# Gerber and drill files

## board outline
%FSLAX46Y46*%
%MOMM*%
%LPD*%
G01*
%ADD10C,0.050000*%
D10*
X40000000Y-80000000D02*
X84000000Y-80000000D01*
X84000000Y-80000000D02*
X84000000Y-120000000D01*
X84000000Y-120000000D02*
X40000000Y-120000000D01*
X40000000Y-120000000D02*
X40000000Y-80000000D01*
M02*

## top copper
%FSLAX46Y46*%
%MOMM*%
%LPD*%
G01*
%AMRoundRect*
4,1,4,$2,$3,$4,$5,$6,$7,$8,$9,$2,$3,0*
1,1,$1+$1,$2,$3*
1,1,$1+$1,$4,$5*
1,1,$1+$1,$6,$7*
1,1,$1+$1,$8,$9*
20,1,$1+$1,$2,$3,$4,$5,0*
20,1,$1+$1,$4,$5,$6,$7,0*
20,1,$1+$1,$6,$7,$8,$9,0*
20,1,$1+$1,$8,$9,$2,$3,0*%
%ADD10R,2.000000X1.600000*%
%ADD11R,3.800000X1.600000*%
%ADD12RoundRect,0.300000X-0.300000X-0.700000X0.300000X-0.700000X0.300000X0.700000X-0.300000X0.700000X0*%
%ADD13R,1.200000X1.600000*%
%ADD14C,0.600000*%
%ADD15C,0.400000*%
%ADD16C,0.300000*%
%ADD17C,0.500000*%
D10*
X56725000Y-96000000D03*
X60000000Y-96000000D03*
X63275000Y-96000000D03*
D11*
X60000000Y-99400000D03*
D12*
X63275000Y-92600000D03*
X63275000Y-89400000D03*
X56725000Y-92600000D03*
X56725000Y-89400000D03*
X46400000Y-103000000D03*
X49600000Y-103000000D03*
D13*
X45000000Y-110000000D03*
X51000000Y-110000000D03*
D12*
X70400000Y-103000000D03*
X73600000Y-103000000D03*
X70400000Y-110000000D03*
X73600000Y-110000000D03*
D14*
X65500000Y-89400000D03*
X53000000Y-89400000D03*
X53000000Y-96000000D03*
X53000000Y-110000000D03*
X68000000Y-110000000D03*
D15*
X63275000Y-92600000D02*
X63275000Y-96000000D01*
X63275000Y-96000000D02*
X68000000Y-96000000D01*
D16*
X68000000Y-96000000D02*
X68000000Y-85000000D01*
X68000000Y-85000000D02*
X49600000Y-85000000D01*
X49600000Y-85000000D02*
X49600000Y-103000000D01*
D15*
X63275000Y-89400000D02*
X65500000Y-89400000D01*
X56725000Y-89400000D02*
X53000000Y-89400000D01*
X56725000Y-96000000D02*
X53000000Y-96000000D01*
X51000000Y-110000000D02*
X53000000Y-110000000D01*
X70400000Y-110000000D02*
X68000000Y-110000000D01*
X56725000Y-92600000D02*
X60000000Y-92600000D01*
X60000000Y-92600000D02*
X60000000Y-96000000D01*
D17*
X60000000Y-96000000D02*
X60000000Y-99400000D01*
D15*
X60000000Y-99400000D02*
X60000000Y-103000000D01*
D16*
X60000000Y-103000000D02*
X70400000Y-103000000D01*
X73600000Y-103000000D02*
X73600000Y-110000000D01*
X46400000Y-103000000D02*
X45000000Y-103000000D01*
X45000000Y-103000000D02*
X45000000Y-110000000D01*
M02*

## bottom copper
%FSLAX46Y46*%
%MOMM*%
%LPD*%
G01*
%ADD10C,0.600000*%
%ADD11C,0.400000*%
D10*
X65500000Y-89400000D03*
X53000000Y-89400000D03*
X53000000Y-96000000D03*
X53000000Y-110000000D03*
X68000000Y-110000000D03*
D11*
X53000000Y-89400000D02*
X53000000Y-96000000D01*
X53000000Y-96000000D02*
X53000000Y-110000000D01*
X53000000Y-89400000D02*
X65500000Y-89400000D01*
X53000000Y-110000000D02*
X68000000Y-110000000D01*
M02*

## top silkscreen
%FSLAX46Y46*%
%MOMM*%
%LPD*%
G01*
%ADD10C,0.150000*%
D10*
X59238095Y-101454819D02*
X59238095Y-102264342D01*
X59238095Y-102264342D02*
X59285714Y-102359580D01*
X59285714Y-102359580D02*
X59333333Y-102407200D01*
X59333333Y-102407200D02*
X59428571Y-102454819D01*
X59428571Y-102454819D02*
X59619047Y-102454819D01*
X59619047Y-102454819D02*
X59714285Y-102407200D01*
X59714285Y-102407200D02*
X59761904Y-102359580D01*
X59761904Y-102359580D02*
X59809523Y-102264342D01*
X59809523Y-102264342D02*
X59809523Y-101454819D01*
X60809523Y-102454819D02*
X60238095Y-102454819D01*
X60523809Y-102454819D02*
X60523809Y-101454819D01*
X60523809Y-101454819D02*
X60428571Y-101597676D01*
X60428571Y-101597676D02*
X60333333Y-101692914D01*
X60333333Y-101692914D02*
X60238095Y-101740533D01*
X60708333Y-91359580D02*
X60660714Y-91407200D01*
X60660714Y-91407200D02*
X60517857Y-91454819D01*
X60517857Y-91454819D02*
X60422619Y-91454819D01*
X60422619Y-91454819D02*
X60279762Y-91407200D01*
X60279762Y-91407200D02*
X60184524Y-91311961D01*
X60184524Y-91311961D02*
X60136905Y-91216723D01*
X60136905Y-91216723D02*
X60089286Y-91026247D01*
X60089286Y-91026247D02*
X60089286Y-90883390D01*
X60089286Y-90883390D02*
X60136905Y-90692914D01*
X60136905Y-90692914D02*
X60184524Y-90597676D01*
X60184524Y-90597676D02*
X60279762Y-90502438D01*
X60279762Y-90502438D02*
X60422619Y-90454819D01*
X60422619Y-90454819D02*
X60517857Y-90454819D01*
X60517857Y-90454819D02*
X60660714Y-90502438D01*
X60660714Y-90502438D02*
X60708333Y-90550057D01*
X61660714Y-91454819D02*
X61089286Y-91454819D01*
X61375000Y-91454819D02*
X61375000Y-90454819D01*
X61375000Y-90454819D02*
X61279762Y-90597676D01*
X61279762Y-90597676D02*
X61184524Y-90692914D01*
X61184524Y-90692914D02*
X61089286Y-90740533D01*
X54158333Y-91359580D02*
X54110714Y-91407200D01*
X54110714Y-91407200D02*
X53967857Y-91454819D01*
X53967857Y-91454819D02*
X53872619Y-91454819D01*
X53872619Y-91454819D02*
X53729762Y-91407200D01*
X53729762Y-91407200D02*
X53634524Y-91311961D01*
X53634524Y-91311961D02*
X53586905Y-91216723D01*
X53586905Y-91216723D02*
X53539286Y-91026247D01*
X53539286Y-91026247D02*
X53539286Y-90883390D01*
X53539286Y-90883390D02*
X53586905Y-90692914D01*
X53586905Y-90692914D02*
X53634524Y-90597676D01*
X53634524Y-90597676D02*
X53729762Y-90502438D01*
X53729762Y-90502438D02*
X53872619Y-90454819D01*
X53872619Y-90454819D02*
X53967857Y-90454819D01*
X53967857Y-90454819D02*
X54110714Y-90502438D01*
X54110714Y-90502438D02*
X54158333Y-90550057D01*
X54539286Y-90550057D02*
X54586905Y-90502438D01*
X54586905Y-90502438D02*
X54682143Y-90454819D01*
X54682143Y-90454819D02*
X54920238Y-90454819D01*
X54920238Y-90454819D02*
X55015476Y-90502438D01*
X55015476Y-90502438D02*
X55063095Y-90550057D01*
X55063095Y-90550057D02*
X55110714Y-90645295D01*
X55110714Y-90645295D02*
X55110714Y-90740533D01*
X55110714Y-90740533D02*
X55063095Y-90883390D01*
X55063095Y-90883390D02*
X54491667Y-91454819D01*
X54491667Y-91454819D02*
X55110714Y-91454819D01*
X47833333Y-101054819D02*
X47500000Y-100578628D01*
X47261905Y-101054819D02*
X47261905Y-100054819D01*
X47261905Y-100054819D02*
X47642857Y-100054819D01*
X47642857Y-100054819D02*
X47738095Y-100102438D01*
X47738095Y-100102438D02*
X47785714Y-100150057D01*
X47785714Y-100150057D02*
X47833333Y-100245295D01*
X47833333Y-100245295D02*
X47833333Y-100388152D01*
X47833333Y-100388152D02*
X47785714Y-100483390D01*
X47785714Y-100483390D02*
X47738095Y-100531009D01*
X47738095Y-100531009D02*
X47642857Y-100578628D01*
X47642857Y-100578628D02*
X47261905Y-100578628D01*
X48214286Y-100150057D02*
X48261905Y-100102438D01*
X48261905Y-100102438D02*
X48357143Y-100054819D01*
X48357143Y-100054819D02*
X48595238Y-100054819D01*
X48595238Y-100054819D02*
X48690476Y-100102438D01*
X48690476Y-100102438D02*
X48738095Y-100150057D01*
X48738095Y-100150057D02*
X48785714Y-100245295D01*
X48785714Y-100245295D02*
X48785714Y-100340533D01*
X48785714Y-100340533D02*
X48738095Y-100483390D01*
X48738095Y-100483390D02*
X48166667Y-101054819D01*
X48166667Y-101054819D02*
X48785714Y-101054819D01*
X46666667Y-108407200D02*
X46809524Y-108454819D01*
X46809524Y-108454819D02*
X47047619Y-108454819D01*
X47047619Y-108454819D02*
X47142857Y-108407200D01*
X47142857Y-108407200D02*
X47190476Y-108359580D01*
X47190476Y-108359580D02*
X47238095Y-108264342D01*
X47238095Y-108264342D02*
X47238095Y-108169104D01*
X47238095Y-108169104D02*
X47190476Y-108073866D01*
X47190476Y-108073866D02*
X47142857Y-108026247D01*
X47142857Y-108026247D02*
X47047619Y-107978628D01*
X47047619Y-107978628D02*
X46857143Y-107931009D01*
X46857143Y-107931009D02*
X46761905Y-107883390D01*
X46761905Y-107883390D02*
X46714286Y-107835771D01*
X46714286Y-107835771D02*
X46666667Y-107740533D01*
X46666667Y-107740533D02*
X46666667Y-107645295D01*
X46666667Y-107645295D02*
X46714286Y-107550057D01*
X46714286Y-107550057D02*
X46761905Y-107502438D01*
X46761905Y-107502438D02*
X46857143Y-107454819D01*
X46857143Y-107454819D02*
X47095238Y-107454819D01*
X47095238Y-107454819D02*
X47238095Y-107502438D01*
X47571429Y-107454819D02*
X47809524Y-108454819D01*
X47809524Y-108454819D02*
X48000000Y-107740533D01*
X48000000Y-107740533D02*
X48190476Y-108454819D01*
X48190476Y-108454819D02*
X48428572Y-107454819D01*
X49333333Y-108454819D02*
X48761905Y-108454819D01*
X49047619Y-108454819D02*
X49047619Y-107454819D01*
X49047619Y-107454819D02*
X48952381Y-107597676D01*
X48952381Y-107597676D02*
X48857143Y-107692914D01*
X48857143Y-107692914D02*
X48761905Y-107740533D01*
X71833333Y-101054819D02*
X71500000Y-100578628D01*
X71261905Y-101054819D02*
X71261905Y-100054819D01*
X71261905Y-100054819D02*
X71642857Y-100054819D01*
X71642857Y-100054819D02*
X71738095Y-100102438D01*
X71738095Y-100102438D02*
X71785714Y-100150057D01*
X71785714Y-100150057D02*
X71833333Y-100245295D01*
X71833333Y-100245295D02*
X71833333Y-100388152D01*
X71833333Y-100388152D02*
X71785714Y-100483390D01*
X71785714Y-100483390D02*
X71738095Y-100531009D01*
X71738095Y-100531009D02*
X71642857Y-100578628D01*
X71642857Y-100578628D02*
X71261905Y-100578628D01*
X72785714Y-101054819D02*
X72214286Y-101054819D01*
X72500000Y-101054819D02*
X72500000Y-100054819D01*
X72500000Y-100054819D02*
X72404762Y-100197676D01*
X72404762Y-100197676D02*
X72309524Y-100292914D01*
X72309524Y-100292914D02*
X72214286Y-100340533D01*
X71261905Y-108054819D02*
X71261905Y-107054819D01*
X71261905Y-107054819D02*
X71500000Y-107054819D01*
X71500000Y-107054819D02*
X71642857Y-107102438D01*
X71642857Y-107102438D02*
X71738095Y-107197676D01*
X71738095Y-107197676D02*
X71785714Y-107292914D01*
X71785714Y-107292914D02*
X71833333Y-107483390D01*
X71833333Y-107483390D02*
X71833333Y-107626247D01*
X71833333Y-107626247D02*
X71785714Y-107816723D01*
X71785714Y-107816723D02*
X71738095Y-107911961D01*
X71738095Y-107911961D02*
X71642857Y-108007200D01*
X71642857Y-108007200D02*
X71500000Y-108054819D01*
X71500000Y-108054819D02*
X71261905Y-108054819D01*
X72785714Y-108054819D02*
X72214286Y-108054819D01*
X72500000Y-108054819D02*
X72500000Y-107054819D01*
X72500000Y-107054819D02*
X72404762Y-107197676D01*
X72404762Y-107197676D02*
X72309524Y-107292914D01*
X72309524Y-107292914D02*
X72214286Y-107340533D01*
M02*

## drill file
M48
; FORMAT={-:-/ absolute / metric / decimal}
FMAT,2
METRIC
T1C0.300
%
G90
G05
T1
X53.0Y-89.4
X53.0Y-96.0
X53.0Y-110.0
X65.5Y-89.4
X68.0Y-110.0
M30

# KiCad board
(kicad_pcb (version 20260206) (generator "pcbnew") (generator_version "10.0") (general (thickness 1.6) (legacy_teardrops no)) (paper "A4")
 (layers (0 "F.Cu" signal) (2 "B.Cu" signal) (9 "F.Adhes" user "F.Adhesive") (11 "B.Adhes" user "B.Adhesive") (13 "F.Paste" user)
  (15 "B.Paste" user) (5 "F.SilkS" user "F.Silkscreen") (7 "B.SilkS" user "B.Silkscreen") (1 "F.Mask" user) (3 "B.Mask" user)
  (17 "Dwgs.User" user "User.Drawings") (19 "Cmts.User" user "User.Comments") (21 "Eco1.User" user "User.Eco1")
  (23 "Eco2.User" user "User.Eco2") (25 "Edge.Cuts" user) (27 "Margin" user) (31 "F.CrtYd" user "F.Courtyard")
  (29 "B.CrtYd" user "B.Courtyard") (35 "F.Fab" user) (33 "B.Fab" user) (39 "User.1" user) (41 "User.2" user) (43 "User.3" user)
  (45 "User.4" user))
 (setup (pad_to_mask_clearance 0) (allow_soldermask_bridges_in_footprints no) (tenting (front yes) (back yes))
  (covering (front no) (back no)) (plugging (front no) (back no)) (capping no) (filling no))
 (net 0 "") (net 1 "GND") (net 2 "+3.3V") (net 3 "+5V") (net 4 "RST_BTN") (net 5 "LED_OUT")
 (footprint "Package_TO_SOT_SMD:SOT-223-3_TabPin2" (layer "F.Cu") (at 60 96)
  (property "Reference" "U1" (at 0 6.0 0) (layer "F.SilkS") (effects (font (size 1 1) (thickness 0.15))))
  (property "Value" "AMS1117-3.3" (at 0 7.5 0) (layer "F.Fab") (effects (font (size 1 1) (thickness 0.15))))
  (pad "1" smd rect (at -3.275 0) (size 2 1.6) (layers "F.Cu" "F.Paste" "F.Mask") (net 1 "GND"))
  (pad "2" smd rect (at 0 0) (size 2 1.6) (layers "F.Cu" "F.Paste" "F.Mask") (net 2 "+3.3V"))
  (pad "3" smd rect (at 3.275 0) (size 2 1.6) (layers "F.Cu" "F.Paste" "F.Mask") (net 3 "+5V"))
  (pad "2" smd rect (at 0 3.4) (size 3.8 1.6) (layers "F.Cu" "F.Paste" "F.Mask") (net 2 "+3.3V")))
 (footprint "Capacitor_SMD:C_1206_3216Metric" (layer "F.Cu") (at 63.275 91 90)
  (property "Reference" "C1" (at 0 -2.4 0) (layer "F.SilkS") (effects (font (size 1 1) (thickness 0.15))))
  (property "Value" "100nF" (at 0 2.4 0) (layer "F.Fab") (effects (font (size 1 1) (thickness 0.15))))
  (pad "1" smd roundrect (at -1.6 0) (size 1.2 2) (layers "F.Cu" "F.Paste" "F.Mask") (roundrect_rratio 0.25) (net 3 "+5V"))
  (pad "2" smd roundrect (at 1.6 0) (size 1.2 2) (layers "F.Cu" "F.Paste" "F.Mask") (roundrect_rratio 0.25) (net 1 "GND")))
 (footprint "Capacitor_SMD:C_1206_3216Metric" (layer "F.Cu") (at 56.725 91 90)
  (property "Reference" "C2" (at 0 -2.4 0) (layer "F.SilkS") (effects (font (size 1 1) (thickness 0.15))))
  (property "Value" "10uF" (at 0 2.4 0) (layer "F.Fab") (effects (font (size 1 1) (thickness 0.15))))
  (pad "1" smd roundrect (at -1.6 0) (size 1.2 2) (layers "F.Cu" "F.Paste" "F.Mask") (roundrect_rratio 0.25) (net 2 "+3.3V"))
  (pad "2" smd roundrect (at 1.6 0) (size 1.2 2) (layers "F.Cu" "F.Paste" "F.Mask") (roundrect_rratio 0.25) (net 1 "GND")))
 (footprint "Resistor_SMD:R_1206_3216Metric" (layer "F.Cu") (at 48 103)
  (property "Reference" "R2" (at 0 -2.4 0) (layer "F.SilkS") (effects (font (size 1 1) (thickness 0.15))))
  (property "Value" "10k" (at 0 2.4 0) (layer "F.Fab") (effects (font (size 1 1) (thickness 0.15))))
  (pad "2" smd roundrect (at -1.6 0) (size 1.2 2) (layers "F.Cu" "F.Paste" "F.Mask") (roundrect_rratio 0.25) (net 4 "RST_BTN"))
  (pad "1" smd roundrect (at 1.6 0) (size 1.2 2) (layers "F.Cu" "F.Paste" "F.Mask") (roundrect_rratio 0.25) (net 3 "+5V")))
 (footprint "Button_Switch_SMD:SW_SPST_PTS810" (layer "F.Cu") (at 48 110)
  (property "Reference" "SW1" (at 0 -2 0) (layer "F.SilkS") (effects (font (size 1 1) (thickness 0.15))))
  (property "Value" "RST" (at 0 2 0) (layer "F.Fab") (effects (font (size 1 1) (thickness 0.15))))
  (pad "1" smd rect (at -3 0) (size 1.2 1.6) (layers "F.Cu" "F.Paste" "F.Mask") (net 4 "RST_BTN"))
  (pad "2" smd rect (at 3 0) (size 1.2 1.6) (layers "F.Cu" "F.Paste" "F.Mask") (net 1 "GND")))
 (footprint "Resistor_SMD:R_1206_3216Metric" (layer "F.Cu") (at 72 103)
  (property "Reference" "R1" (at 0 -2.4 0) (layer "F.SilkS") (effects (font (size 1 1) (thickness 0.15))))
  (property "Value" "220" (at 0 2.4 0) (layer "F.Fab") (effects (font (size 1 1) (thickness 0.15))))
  (pad "1" smd roundrect (at -1.6 0) (size 1.2 2) (layers "F.Cu" "F.Paste" "F.Mask") (roundrect_rratio 0.25) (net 2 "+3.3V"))
  (pad "2" smd roundrect (at 1.6 0) (size 1.2 2) (layers "F.Cu" "F.Paste" "F.Mask") (roundrect_rratio 0.25) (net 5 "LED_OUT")))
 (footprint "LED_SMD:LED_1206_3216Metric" (layer "F.Cu") (at 72 110)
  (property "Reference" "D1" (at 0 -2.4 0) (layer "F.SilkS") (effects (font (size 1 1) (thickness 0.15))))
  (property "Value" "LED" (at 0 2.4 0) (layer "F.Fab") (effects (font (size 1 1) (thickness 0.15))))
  (pad "2" smd roundrect (at -1.6 0) (size 1.2 2) (layers "F.Cu" "F.Paste" "F.Mask") (roundrect_rratio 0.25) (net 1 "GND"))
  (pad "1" smd roundrect (at 1.6 0) (size 1.2 2) (layers "F.Cu" "F.Paste" "F.Mask") (roundrect_rratio 0.25) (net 5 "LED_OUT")))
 (segment (start 63.275 92.6) (end 63.275 96) (width 0.4) (layer "F.Cu") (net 3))
 (segment (start 63.275 96) (end 68 96) (width 0.4) (layer "F.Cu") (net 3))
 (segment (start 68 96) (end 68 85) (width 0.3) (layer "F.Cu") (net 3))
 (segment (start 68 85) (end 49.6 85) (width 0.3) (layer "F.Cu") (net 3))
 (segment (start 49.6 85) (end 49.6 103) (width 0.3) (layer "F.Cu") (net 3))
 (segment (start 63.275 89.4) (end 65.5 89.4) (width 0.4) (layer "F.Cu") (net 1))
 (via (at 65.5 89.4) (size 0.6) (drill 0.3) (layers "F.Cu" "B.Cu") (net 1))
 (segment (start 56.725 89.4) (end 53 89.4) (width 0.4) (layer "F.Cu") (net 1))
 (via (at 53 89.4) (size 0.6) (drill 0.3) (layers "F.Cu" "B.Cu") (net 1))
 (segment (start 56.725 96) (end 53 96) (width 0.4) (layer "F.Cu") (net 1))
 (via (at 53 96) (size 0.6) (drill 0.3) (layers "F.Cu" "B.Cu") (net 1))
 (segment (start 51 110) (end 53 110) (width 0.4) (layer "F.Cu") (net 1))
 (via (at 53 110) (size 0.6) (drill 0.3) (layers "F.Cu" "B.Cu") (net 1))
 (segment (start 70.4 110) (end 68 110) (width 0.4) (layer "F.Cu") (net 1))
 (via (at 68 110) (size 0.6) (drill 0.3) (layers "F.Cu" "B.Cu") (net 1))
 (segment (start 53 89.4) (end 53 96) (width 0.4) (layer "B.Cu") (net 1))
 (segment (start 53 96) (end 53 110) (width 0.4) (layer "B.Cu") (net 1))
 (segment (start 53 89.4) (end 65.5 89.4) (width 0.4) (layer "B.Cu") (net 1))
 (segment (start 53 110) (end 68 110) (width 0.4) (layer "B.Cu") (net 1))
 (segment (start 56.725 92.6) (end 60 92.6) (width 0.4) (layer "F.Cu") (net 2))
 (segment (start 60 92.6) (end 60 96) (width 0.4) (layer "F.Cu") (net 2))
 (segment (start 60 96) (end 60 99.4) (width 0.5) (layer "F.Cu") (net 2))
 (segment (start 60 99.4) (end 60 103) (width 0.4) (layer "F.Cu") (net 2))
 (segment (start 60 103) (end 70.4 103) (width 0.3) (layer "F.Cu") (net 2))
 (segment (start 73.6 103) (end 73.6 110) (width 0.3) (layer "F.Cu") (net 5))
 (segment (start 46.4 103) (end 45 103) (width 0.3) (layer "F.Cu") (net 4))
 (segment (start 45 103) (end 45 110) (width 0.3) (layer "F.Cu") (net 4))
 (gr_line (start 40 80) (end 84 80) (stroke (width 0.05) (type solid)) (layer "Edge.Cuts"))
 (gr_line (start 84 80) (end 84 120) (stroke (width 0.05) (type solid)) (layer "Edge.Cuts"))
 (gr_line (start 84 120) (end 40 120) (stroke (width 0.05) (type solid)) (layer "Edge.Cuts"))
 (gr_line (start 40 120) (end 40 80) (stroke (width 0.05) (type solid)) (layer "Edge.Cuts")))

